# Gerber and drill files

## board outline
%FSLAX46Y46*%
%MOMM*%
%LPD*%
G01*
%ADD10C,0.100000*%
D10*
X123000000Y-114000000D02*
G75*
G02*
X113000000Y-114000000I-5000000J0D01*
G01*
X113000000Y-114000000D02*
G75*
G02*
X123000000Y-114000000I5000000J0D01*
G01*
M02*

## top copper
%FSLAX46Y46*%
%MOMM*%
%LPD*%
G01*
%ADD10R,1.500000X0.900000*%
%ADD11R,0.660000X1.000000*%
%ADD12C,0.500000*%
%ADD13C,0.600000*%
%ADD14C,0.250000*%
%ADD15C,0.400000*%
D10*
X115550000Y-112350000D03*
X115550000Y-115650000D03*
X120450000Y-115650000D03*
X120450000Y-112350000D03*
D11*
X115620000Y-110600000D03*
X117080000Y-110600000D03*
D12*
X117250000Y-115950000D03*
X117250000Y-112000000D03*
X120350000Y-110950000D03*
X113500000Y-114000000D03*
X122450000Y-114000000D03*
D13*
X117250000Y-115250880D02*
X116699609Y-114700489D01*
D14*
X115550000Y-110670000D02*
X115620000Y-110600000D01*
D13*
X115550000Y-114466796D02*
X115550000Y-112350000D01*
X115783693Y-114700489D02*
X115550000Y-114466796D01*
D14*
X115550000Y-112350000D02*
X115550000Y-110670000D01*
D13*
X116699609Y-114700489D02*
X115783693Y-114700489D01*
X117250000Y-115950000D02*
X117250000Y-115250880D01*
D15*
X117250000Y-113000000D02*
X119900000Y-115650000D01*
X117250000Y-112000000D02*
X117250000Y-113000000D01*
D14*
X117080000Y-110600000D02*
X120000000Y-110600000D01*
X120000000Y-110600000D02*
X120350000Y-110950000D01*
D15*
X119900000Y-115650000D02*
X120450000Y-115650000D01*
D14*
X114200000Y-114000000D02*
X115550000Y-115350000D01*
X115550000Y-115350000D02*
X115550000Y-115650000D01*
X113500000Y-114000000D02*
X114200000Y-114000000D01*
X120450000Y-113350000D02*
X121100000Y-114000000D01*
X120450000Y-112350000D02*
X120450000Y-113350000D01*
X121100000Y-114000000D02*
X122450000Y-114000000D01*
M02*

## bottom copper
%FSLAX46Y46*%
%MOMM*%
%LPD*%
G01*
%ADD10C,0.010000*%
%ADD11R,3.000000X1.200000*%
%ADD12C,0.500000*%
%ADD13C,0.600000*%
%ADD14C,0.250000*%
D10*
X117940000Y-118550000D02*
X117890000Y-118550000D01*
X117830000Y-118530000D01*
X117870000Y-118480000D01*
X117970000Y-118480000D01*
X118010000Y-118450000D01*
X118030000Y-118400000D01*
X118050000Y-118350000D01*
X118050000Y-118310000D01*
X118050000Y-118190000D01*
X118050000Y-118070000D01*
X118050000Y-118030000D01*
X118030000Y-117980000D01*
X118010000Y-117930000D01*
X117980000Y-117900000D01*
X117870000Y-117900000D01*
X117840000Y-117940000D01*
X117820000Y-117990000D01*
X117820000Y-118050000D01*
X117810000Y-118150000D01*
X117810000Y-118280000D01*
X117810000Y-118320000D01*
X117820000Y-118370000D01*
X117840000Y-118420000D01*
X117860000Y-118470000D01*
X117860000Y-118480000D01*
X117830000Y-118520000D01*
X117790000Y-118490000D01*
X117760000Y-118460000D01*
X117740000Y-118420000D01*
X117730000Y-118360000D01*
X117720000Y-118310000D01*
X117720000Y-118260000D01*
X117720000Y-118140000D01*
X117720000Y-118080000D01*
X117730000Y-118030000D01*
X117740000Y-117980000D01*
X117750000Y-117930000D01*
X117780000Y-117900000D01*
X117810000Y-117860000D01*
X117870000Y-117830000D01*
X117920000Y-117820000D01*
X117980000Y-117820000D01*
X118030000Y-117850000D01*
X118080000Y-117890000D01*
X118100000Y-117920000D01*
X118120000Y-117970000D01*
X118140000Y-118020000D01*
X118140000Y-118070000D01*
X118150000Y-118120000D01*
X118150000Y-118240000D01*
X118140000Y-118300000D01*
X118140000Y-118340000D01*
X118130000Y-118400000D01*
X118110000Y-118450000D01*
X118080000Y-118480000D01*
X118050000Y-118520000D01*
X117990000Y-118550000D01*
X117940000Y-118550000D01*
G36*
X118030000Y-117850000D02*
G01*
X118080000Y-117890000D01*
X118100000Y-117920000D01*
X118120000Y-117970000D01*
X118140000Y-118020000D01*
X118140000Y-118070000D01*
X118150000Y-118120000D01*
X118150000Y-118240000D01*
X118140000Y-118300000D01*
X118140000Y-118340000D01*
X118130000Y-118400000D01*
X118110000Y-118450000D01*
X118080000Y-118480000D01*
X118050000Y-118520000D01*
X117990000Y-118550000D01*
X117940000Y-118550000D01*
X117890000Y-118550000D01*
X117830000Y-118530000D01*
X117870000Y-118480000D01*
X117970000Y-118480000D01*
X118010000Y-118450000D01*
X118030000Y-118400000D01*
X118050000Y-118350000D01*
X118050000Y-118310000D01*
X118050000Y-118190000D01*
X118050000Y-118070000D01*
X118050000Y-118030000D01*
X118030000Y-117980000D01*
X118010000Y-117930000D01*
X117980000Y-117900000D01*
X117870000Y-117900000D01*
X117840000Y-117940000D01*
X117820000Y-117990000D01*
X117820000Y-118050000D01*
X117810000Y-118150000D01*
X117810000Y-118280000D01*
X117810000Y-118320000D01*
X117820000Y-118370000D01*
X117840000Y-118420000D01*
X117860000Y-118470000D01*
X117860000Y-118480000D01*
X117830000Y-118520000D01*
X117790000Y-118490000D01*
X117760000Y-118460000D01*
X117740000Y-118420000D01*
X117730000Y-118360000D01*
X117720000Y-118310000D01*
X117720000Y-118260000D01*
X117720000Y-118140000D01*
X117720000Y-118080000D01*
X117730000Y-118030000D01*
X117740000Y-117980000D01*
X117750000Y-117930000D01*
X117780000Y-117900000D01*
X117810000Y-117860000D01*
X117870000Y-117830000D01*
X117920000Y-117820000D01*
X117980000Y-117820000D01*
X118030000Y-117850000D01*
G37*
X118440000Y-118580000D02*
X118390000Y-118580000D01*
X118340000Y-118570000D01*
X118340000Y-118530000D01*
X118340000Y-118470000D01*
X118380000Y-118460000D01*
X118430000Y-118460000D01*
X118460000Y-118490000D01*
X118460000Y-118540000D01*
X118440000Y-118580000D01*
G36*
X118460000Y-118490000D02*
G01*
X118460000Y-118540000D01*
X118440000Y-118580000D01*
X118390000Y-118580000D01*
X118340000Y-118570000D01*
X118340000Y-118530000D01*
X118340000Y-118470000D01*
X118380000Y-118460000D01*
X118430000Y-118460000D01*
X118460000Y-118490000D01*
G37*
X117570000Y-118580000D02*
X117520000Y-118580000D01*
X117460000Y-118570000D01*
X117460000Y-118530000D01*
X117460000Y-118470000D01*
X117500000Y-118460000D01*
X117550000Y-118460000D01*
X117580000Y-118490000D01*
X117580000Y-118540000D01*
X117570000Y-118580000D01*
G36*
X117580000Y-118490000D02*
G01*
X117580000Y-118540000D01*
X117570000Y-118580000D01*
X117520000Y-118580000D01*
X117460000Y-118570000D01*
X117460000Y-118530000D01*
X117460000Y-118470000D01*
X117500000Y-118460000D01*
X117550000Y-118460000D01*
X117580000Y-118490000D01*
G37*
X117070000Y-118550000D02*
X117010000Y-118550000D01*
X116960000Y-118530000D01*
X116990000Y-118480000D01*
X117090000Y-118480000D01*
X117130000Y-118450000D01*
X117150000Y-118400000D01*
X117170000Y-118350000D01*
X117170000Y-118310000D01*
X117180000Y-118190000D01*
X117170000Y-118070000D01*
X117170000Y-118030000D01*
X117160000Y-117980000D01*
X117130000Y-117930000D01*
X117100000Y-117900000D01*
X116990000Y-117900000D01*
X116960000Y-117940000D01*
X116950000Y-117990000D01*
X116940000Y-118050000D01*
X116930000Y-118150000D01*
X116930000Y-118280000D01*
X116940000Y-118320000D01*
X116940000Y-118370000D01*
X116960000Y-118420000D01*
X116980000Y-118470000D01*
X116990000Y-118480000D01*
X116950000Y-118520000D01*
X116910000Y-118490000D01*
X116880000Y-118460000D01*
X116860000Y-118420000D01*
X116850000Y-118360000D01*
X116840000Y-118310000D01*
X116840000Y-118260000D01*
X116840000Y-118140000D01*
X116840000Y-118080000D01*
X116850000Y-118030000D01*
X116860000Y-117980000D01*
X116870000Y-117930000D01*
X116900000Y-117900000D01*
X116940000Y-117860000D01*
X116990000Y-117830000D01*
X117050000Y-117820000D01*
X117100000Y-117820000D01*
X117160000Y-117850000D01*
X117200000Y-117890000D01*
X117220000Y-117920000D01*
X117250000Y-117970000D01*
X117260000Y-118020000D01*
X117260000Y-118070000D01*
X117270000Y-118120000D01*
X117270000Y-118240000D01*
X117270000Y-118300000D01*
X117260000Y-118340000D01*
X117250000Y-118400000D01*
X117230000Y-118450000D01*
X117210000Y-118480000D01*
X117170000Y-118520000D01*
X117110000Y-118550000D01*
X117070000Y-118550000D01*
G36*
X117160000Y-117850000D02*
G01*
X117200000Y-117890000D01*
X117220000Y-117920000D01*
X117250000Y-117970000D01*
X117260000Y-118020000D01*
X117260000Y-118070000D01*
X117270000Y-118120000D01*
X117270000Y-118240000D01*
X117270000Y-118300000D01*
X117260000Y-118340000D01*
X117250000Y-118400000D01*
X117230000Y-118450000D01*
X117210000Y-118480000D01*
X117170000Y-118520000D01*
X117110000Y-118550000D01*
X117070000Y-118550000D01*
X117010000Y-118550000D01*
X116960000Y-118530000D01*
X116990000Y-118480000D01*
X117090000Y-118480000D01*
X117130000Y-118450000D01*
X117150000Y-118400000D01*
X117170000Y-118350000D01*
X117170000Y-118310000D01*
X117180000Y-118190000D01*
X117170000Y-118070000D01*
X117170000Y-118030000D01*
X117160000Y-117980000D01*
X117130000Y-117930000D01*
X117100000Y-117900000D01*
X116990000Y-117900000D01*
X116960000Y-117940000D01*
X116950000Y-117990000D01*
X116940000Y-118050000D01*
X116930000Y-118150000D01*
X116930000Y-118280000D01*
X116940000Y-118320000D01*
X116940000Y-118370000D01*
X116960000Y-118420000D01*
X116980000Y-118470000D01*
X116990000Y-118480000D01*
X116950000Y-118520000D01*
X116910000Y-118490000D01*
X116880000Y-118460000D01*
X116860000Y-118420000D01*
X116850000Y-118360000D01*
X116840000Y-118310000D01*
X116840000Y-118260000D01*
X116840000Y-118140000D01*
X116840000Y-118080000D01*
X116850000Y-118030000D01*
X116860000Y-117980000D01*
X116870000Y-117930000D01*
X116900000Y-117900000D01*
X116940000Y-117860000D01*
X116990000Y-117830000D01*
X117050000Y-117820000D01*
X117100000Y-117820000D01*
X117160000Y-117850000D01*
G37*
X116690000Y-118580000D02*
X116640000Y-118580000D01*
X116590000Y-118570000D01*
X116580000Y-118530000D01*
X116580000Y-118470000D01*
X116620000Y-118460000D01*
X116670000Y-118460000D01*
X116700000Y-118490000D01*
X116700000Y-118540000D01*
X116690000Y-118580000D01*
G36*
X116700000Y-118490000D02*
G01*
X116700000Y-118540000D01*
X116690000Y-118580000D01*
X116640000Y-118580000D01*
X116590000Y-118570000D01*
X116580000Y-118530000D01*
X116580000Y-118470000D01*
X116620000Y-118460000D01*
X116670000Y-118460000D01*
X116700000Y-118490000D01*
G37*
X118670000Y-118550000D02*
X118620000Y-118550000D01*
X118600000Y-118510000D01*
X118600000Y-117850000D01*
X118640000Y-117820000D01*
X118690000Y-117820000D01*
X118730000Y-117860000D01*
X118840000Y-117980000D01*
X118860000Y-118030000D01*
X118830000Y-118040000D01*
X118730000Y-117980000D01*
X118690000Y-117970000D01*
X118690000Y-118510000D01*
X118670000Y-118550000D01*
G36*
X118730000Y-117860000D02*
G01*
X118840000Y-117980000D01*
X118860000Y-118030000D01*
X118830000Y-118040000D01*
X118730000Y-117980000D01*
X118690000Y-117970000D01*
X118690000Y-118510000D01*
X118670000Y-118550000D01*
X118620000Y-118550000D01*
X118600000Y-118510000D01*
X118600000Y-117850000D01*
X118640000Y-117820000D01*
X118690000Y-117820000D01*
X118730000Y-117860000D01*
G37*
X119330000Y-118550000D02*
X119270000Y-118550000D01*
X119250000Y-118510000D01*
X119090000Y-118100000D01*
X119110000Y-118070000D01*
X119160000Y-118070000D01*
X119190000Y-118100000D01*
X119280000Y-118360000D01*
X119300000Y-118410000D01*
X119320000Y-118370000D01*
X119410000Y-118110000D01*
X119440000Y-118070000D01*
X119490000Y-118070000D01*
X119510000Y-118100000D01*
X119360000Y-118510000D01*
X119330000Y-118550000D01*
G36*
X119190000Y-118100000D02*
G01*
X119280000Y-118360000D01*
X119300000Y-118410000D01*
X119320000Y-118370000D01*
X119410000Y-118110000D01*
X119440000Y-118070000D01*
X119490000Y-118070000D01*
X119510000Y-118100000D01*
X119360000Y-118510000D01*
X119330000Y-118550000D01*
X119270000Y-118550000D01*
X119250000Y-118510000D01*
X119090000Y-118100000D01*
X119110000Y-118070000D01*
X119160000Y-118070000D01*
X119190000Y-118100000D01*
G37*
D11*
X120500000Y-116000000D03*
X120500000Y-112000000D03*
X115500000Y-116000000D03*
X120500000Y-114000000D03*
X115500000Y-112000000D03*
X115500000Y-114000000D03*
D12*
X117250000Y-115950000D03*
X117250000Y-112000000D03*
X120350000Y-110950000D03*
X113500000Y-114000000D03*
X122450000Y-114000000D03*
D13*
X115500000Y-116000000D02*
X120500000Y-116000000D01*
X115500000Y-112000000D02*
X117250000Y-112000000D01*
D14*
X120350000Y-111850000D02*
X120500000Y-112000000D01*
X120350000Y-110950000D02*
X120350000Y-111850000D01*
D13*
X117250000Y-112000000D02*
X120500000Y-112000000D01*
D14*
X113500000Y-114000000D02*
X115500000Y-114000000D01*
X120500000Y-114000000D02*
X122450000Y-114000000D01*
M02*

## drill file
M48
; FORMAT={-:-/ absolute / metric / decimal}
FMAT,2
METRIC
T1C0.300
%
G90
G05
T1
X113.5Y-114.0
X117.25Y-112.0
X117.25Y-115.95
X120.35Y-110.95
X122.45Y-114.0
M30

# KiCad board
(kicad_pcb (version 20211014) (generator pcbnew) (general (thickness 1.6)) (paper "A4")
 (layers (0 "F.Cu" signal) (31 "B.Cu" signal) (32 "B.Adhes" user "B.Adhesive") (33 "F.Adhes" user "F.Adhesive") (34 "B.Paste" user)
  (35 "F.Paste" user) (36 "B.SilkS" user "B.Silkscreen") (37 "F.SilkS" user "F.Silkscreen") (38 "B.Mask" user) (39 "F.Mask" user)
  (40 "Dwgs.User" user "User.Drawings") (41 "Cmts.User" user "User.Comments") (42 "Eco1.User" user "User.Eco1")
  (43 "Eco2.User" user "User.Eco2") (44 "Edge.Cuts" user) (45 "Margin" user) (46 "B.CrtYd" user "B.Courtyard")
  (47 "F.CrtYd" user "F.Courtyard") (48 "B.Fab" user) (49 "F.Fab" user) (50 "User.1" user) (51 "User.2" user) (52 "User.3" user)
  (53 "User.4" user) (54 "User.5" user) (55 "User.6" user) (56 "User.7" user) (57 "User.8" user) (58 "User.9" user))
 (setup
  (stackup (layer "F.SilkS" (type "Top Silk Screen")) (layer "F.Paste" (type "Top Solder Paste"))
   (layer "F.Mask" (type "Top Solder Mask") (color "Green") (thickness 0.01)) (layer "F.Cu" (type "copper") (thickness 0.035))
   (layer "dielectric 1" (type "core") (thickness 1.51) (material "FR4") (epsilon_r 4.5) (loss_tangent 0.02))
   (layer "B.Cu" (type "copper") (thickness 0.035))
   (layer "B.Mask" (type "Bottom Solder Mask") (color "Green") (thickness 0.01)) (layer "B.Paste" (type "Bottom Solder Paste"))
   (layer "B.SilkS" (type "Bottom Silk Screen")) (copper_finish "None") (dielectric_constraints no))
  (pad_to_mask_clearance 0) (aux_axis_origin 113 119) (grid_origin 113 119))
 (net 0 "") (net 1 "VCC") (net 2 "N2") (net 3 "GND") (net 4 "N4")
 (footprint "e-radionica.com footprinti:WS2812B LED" (layer "F.Cu") (at 118 114)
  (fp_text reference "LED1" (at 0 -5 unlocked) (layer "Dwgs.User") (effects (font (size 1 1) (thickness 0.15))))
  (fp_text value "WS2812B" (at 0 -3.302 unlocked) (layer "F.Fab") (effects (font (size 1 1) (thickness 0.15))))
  (pad "1" smd rect (at -2.45 -1.65) (size 1.5 0.9) (layers "F.Cu" "F.Paste" "F.Mask") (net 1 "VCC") (solder_mask_margin 0.1))
  (pad "2" smd rect (at -2.45 1.65) (size 1.5 0.9) (layers "F.Cu" "F.Paste" "F.Mask") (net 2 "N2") (solder_mask_margin 0.1))
  (pad "3" smd rect (at 2.45 1.65) (size 1.5 0.9) (layers "F.Cu" "F.Paste" "F.Mask") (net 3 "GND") (solder_mask_margin 0.1))
  (pad "4" smd rect (at 2.45 -1.65) (size 1.5 0.9) (layers "F.Cu" "F.Paste" "F.Mask") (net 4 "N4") (solder_mask_margin 0.1)))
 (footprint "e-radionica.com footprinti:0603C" (layer "F.Cu") (at 116.35 110.6)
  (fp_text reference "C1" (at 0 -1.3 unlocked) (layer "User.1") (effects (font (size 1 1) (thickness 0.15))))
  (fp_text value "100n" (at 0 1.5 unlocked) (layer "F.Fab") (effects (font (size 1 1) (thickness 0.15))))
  (pad "1" smd rect locked (at -0.73 0) (size 0.66 1) (layers "F.Cu" "F.Paste" "F.Mask") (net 1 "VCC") (solder_mask_margin 0.1))
  (pad "2" smd rect locked (at 0.73 0) (size 0.66 1) (layers "F.Cu" "F.Paste" "F.Mask") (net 3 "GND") (solder_mask_margin 0.1)))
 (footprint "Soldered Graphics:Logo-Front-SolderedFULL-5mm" (layer "F.Cu") (at 118 117.62)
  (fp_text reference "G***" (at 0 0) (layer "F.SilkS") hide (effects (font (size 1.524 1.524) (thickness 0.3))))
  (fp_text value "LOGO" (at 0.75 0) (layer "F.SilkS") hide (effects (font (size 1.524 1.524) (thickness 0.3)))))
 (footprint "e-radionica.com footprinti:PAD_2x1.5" (layer "B.Cu") (at 121 116 180)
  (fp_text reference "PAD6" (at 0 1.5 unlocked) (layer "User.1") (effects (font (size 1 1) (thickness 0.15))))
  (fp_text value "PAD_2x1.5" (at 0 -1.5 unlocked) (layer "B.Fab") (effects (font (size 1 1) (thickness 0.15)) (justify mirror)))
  (pad "1" smd rect (at 0.5 0 180) (size 3 1.2) (layers "B.Cu" "B.Paste" "B.Mask") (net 1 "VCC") (solder_mask_margin 0.1)))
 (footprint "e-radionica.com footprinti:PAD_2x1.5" (layer "B.Cu") (at 121 112 180)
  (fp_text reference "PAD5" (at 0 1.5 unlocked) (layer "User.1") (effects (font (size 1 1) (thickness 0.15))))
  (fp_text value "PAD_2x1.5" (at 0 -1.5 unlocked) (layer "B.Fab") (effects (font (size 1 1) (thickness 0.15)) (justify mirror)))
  (pad "1" smd rect (at 0.5 0 180) (size 3 1.2) (layers "B.Cu" "B.Paste" "B.Mask") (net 3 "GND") (solder_mask_margin 0.1)))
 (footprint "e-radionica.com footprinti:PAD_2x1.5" (layer "B.Cu") (at 115 116 180)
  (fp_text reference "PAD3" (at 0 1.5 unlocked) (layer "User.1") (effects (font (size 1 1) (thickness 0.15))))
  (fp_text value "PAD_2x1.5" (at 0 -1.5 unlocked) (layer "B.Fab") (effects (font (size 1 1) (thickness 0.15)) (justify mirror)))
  (pad "1" smd rect (at -0.5 0 180) (size 3 1.2) (layers "B.Cu" "B.Paste" "B.Mask") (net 1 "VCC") (solder_mask_margin 0.1)))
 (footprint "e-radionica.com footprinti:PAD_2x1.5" (layer "B.Cu") (at 121 114 180)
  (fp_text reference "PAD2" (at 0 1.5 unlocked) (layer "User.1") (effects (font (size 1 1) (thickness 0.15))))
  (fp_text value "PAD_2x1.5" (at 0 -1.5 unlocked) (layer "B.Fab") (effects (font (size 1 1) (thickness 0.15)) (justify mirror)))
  (pad "1" smd rect (at 0.5 0 180) (size 3 1.2) (layers "B.Cu" "B.Paste" "B.Mask") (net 4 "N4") (solder_mask_margin 0.1)))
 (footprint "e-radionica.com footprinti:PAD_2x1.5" (layer "B.Cu") (at 115.5 112 180)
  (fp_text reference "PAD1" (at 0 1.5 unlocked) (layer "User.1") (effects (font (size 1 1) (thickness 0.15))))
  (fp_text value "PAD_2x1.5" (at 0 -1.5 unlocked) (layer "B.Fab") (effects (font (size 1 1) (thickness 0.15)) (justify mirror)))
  (pad "1" smd rect (at 0 0 180) (size 3 1.2) (layers "B.Cu" "B.Paste" "B.Mask") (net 3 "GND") (solder_mask_margin 0.1)))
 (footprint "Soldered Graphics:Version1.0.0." (layer "B.Cu") (at 118 118.2 180)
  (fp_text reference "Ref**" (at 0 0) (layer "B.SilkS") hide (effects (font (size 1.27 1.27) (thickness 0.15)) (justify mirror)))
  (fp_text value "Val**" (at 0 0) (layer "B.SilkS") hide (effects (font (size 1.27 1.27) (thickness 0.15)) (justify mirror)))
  (fp_poly
   (pts (xy 0.06 -0.35) (xy 0.11 -0.35) (xy 0.17 -0.33) (xy 0.13 -0.28) (xy 0.03 -0.28) (xy -0.01 -0.25) (xy -0.03 -0.2) (xy -0.05 -0.15)
    (xy -0.05 -0.11) (xy -0.05 0.01) (xy -0.05 0.13) (xy -0.05 0.17) (xy -0.03 0.22) (xy -0.01 0.27) (xy 0.02 0.3) (xy 0.13 0.3)
    (xy 0.16 0.26) (xy 0.18 0.21) (xy 0.18 0.15) (xy 0.19 0.05) (xy 0.19 -0.08) (xy 0.19 -0.12) (xy 0.18 -0.17) (xy 0.16 -0.22)
    (xy 0.14 -0.27) (xy 0.14 -0.28) (xy 0.17 -0.32) (xy 0.21 -0.29) (xy 0.24 -0.26) (xy 0.26 -0.22) (xy 0.27 -0.16) (xy 0.28 -0.11)
    (xy 0.28 -0.06) (xy 0.28 0.06) (xy 0.28 0.12) (xy 0.27 0.17) (xy 0.26 0.22) (xy 0.25 0.27) (xy 0.22 0.3) (xy 0.19 0.34) (xy 0.13 0.37)
    (xy 0.08 0.38) (xy 0.02 0.38) (xy -0.03 0.35) (xy -0.08 0.31) (xy -0.1 0.28) (xy -0.12 0.23) (xy -0.14 0.18) (xy -0.14 0.13)
    (xy -0.15 0.08) (xy -0.15 -0.04) (xy -0.14 -0.1) (xy -0.14 -0.14) (xy -0.13 -0.2) (xy -0.11 -0.25) (xy -0.08 -0.28) (xy -0.05 -0.32)
    (xy 0.01 -0.35) (xy 0.06 -0.35))
   (layer "B.Cu") (width 0.01) (fill solid))
  (fp_poly
   (pts (xy -0.44 -0.38) (xy -0.39 -0.38) (xy -0.34 -0.37) (xy -0.34 -0.33) (xy -0.34 -0.27) (xy -0.38 -0.26) (xy -0.43 -0.26)
    (xy -0.46 -0.29) (xy -0.46 -0.34) (xy -0.44 -0.38))
   (layer "B.Cu") (width 0.01) (fill solid))
  (fp_poly
   (pts (xy 0.43 -0.38) (xy 0.48 -0.38) (xy 0.54 -0.37) (xy 0.54 -0.33) (xy 0.54 -0.27) (xy 0.5 -0.26) (xy 0.45 -0.26) (xy 0.42 -0.29)
    (xy 0.42 -0.34) (xy 0.43 -0.38))
   (layer "B.Cu") (width 0.01) (fill solid))
  (fp_poly
   (pts (xy 0.93 -0.35) (xy 0.99 -0.35) (xy 1.04 -0.33) (xy 1.01 -0.28) (xy 0.91 -0.28) (xy 0.87 -0.25) (xy 0.85 -0.2) (xy 0.83 -0.15)
    (xy 0.83 -0.11) (xy 0.82 0.01) (xy 0.83 0.13) (xy 0.83 0.17) (xy 0.84 0.22) (xy 0.87 0.27) (xy 0.9 0.3) (xy 1.01 0.3) (xy 1.04 0.26)
    (xy 1.05 0.21) (xy 1.06 0.15) (xy 1.07 0.05) (xy 1.07 -0.08) (xy 1.06 -0.12) (xy 1.06 -0.17) (xy 1.04 -0.22) (xy 1.02 -0.27)
    (xy 1.01 -0.28) (xy 1.05 -0.32) (xy 1.09 -0.29) (xy 1.12 -0.26) (xy 1.14 -0.22) (xy 1.15 -0.16) (xy 1.16 -0.11) (xy 1.16 -0.06)
    (xy 1.16 0.06) (xy 1.16 0.12) (xy 1.15 0.17) (xy 1.14 0.22) (xy 1.13 0.27) (xy 1.1 0.3) (xy 1.06 0.34) (xy 1.01 0.37) (xy 0.95 0.38)
    (xy 0.9 0.38) (xy 0.84 0.35) (xy 0.8 0.31) (xy 0.78 0.28) (xy 0.75 0.23) (xy 0.74 0.18) (xy 0.74 0.13) (xy 0.73 0.08) (xy 0.73 -0.04)
    (xy 0.73 -0.1) (xy 0.74 -0.14) (xy 0.75 -0.2) (xy 0.77 -0.25) (xy 0.79 -0.28) (xy 0.83 -0.32) (xy 0.89 -0.35) (xy 0.93 -0.35))
   (layer "B.Cu") (width 0.01) (fill solid))
  (fp_poly
   (pts (xy 1.31 -0.38) (xy 1.36 -0.38) (xy 1.41 -0.37) (xy 1.42 -0.33) (xy 1.42 -0.27) (xy 1.38 -0.26) (xy 1.33 -0.26) (xy 1.3 -0.29)
    (xy 1.3 -0.34) (xy 1.31 -0.38))
   (layer "B.Cu") (width 0.01) (fill solid))
  (fp_poly
   (pts (xy -0.67 -0.35) (xy -0.62 -0.35) (xy -0.6 -0.31) (xy -0.6 0.35) (xy -0.64 0.38) (xy -0.69 0.38) (xy -0.73 0.34) (xy -0.84 0.22)
    (xy -0.86 0.17) (xy -0.83 0.16) (xy -0.73 0.22) (xy -0.69 0.23) (xy -0.69 -0.31) (xy -0.67 -0.35))
   (layer "B.Cu") (width 0.01) (fill solid))
  (fp_poly
   (pts (xy -1.33 -0.35) (xy -1.27 -0.35) (xy -1.25 -0.31) (xy -1.09 0.1) (xy -1.11 0.13) (xy -1.16 0.13) (xy -1.19 0.1) (xy -1.28 -0.16)
    (xy -1.3 -0.21) (xy -1.32 -0.17) (xy -1.41 0.09) (xy -1.44 0.13) (xy -1.49 0.13) (xy -1.51 0.1) (xy -1.36 -0.31) (xy -1.33 -0.35))
   (layer "B.Cu") (width 0.01) (fill solid)))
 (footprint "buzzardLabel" (layer "B.Cu") (at 118 112 180)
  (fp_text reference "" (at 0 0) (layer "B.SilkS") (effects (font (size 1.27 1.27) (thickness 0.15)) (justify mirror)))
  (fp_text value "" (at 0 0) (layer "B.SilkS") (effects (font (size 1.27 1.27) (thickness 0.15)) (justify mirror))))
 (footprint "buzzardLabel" (layer "B.Cu") (at 118 116 180)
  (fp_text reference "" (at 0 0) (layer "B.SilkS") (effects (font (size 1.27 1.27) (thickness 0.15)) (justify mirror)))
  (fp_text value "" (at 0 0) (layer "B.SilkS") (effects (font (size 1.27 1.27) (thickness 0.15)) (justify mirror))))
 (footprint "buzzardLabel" (layer "B.Cu") (at 118 114 180)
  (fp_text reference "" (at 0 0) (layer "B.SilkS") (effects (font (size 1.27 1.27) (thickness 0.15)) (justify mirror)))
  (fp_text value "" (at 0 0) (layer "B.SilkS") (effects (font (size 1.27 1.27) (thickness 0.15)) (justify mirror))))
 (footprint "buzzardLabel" (layer "B.Cu") (at 118 110.3 180)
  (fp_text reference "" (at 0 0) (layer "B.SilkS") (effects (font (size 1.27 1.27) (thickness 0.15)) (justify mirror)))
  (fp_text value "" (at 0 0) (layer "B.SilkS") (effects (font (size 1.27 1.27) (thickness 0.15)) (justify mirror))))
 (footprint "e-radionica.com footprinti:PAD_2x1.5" (layer "B.Cu") (at 115 114 -90)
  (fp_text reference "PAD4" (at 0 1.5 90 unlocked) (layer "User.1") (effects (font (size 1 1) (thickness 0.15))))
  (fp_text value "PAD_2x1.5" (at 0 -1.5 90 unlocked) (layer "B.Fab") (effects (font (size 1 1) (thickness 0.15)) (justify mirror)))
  (pad "1" smd rect (at 0 -0.5 180) (size 3 1.2) (layers "B.Cu" "B.Paste" "B.Mask") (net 2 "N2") (solder_mask_margin 0.1)))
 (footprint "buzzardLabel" (layer "B.Cu") (at 118 117.8 180)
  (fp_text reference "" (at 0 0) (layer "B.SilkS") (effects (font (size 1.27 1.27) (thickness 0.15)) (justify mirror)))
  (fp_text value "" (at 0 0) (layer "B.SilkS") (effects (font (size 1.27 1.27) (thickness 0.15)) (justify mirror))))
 (gr_circle (center 118 114) (end 118 109) (layer "Edge.Cuts") (width 0.1) (fill none))
 (segment (start 117.25 115.25088) (end 116.699609 114.700489) (width 0.6) (layer "F.Cu") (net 1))
 (segment (start 115.55 110.67) (end 115.62 110.6) (width 0.25) (layer "F.Cu") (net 1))
 (segment (start 115.55 114.466796) (end 115.55 112.35) (width 0.6) (layer "F.Cu") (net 1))
 (segment (start 115.783693 114.700489) (end 115.55 114.466796) (width 0.6) (layer "F.Cu") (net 1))
 (segment (start 115.55 112.35) (end 115.55 110.67) (width 0.25) (layer "F.Cu") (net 1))
 (segment (start 116.699609 114.700489) (end 115.783693 114.700489) (width 0.6) (layer "F.Cu") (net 1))
 (segment (start 117.25 115.95) (end 117.25 115.25088) (width 0.6) (layer "F.Cu") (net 1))
 (via (at 117.25 115.95) (size 0.5) (drill 0.3) (layers "F.Cu" "B.Cu") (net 1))
 (segment (start 115.5 116) (end 120.5 116) (width 0.6) (layer "B.Cu") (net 1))
 (segment (start 117.25 113) (end 119.9 115.65) (width 0.4) (layer "F.Cu") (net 3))
 (segment (start 117.25 112) (end 117.25 113) (width 0.4) (layer "F.Cu") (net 3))
 (segment (start 117.08 110.6) (end 120 110.6) (width 0.25) (layer "F.Cu") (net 3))
 (segment (start 120 110.6) (end 120.35 110.95) (width 0.25) (layer "F.Cu") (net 3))
 (segment (start 119.9 115.65) (end 120.45 115.65) (width 0.4) (layer "F.Cu") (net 3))
 (via (at 117.25 112) (size 0.5) (drill 0.3) (layers "F.Cu" "B.Cu") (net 3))
 (via (at 120.35 110.95) (size 0.5) (drill 0.3) (layers "F.Cu" "B.Cu") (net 3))
 (segment (start 115.5 112) (end 117.25 112) (width 0.6) (layer "B.Cu") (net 3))
 (segment (start 120.35 111.85) (end 120.5 112) (width 0.25) (layer "B.Cu") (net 3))
 (segment (start 120.35 110.95) (end 120.35 111.85) (width 0.25) (layer "B.Cu") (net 3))
 (segment (start 117.25 112) (end 120.5 112) (width 0.6) (layer "B.Cu") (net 3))
 (segment (start 114.2 114) (end 115.55 115.35) (width 0.25) (layer "F.Cu") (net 2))
 (segment (start 115.55 115.35) (end 115.55 115.65) (width 0.25) (layer "F.Cu") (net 2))
 (segment (start 113.5 114) (end 114.2 114) (width 0.25) (layer "F.Cu") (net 2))
 (via (at 113.5 114) (size 0.5) (drill 0.3) (layers "F.Cu" "B.Cu") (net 2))
 (segment (start 113.5 114) (end 115.5 114) (width 0.25) (layer "B.Cu") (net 2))
 (segment (start 120.45 113.35) (end 121.1 114) (width 0.25) (layer "F.Cu") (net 4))
 (segment (start 120.45 112.35) (end 120.45 113.35) (width 0.25) (layer "F.Cu") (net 4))
 (segment (start 121.1 114) (end 122.45 114) (width 0.25) (layer "F.Cu") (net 4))
 (via (at 122.45 114) (size 0.5) (drill 0.3) (layers "F.Cu" "B.Cu") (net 4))
 (segment (start 120.5 114) (end 122.45 114) (width 0.25) (layer "B.Cu") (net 4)))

